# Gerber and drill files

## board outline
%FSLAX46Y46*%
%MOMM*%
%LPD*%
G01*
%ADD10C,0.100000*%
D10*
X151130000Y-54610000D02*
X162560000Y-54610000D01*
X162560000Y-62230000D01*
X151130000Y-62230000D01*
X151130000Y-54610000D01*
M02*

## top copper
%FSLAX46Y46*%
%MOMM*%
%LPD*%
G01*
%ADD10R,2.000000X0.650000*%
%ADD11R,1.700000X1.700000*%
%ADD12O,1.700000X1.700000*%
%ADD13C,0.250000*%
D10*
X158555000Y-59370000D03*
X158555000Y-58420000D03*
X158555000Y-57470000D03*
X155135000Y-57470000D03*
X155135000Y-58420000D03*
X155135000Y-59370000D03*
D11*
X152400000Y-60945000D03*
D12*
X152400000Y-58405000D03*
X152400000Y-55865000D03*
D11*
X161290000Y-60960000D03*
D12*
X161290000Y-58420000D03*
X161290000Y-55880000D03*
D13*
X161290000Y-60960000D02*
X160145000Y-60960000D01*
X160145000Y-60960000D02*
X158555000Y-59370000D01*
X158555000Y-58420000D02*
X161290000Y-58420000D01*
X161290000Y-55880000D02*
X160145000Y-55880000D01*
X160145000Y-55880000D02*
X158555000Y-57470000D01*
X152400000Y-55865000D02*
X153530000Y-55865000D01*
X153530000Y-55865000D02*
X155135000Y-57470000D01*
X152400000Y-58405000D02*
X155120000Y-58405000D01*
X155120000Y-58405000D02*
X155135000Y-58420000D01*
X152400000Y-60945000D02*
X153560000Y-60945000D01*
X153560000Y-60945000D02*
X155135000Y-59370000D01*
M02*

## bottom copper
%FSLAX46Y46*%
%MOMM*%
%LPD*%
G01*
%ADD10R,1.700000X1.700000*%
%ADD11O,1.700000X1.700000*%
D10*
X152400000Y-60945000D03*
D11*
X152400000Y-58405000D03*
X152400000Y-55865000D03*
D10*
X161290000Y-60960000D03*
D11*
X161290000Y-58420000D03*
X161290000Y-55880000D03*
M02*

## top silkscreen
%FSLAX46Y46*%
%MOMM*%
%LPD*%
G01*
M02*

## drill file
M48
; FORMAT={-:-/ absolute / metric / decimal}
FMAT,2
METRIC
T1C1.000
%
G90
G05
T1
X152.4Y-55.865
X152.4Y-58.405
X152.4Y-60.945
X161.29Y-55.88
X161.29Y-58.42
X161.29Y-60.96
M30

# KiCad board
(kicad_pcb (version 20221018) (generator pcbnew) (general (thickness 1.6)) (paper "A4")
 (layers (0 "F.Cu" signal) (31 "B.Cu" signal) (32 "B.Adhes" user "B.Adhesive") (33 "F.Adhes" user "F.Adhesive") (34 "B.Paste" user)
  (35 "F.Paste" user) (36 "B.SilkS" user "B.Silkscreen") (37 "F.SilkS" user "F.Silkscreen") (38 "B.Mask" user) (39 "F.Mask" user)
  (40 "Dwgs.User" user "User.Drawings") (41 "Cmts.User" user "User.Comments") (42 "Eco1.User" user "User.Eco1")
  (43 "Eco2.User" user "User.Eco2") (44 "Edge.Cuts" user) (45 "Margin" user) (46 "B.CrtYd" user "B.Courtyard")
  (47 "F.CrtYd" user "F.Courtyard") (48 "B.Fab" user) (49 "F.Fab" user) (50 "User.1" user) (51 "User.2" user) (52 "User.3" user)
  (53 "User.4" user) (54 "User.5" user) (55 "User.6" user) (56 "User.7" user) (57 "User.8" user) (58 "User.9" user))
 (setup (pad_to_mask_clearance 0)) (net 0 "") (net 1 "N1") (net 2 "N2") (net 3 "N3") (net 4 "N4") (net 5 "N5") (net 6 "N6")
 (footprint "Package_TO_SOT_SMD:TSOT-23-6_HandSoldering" (layer "F.Cu") (at 156.845 58.42 180)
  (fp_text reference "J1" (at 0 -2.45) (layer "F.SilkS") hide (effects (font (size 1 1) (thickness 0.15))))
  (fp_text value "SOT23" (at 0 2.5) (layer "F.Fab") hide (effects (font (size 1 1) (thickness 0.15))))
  (pad "1" smd rect (at -1.71 -0.95 180) (size 2 0.65) (layers "F.Cu" "F.Paste" "F.Mask") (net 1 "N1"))
  (pad "2" smd rect (at -1.71 0 180) (size 2 0.65) (layers "F.Cu" "F.Paste" "F.Mask") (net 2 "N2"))
  (pad "3" smd rect (at -1.71 0.95 180) (size 2 0.65) (layers "F.Cu" "F.Paste" "F.Mask") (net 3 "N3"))
  (pad "4" smd rect (at 1.71 0.95 180) (size 2 0.65) (layers "F.Cu" "F.Paste" "F.Mask") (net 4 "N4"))
  (pad "5" smd rect (at 1.71 0 180) (size 2 0.65) (layers "F.Cu" "F.Paste" "F.Mask") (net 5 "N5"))
  (pad "6" smd rect (at 1.71 -0.95 180) (size 2 0.65) (layers "F.Cu" "F.Paste" "F.Mask") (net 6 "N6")))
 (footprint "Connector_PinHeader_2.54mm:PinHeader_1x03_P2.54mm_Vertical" (layer "F.Cu") (at 152.4 60.945 180)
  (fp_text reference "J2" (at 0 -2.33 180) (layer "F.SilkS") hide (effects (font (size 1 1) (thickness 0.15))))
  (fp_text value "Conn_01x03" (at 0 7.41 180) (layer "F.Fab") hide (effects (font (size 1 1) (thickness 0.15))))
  (pad "1" thru_hole rect (at 0 0 180) (size 1.7 1.7) (drill 1) (layers "*.Cu" "*.Mask") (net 6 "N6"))
  (pad "2" thru_hole oval (at 0 2.54 180) (size 1.7 1.7) (drill 1) (layers "*.Cu" "*.Mask") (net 5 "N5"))
  (pad "3" thru_hole oval (at 0 5.08 180) (size 1.7 1.7) (drill 1) (layers "*.Cu" "*.Mask") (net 4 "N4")))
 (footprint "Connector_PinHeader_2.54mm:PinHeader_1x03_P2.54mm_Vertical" (layer "F.Cu") (at 161.29 60.96 180)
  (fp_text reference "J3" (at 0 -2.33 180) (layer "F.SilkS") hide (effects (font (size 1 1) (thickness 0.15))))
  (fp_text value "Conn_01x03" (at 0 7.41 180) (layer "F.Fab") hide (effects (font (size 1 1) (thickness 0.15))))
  (pad "1" thru_hole rect (at 0 0 180) (size 1.7 1.7) (drill 1) (layers "*.Cu" "*.Mask") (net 1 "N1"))
  (pad "2" thru_hole oval (at 0 2.54 180) (size 1.7 1.7) (drill 1) (layers "*.Cu" "*.Mask") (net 2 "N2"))
  (pad "3" thru_hole oval (at 0 5.08 180) (size 1.7 1.7) (drill 1) (layers "*.Cu" "*.Mask") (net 3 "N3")))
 (gr_rect (start 151.13 54.61) (end 162.56 62.23) (stroke (width 0.1) (type default)) (fill none) (layer "Edge.Cuts"))
 (segment (start 161.29 60.96) (end 160.145 60.96) (width 0.25) (layer "F.Cu") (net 1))
 (segment (start 160.145 60.96) (end 158.555 59.37) (width 0.25) (layer "F.Cu") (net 1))
 (segment (start 158.555 58.42) (end 161.29 58.42) (width 0.25) (layer "F.Cu") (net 2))
 (segment (start 161.29 55.88) (end 160.145 55.88) (width 0.25) (layer "F.Cu") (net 3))
 (segment (start 160.145 55.88) (end 158.555 57.47) (width 0.25) (layer "F.Cu") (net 3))
 (segment (start 152.4 55.865) (end 153.53 55.865) (width 0.25) (layer "F.Cu") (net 4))
 (segment (start 153.53 55.865) (end 155.135 57.47) (width 0.25) (layer "F.Cu") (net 4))
 (segment (start 152.4 58.405) (end 155.12 58.405) (width 0.25) (layer "F.Cu") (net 5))
 (segment (start 155.12 58.405) (end 155.135 58.42) (width 0.25) (layer "F.Cu") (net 5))
 (segment (start 152.4 60.945) (end 153.56 60.945) (width 0.25) (layer "F.Cu") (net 6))
 (segment (start 153.56 60.945) (end 155.135 59.37) (width 0.25) (layer "F.Cu") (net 6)))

